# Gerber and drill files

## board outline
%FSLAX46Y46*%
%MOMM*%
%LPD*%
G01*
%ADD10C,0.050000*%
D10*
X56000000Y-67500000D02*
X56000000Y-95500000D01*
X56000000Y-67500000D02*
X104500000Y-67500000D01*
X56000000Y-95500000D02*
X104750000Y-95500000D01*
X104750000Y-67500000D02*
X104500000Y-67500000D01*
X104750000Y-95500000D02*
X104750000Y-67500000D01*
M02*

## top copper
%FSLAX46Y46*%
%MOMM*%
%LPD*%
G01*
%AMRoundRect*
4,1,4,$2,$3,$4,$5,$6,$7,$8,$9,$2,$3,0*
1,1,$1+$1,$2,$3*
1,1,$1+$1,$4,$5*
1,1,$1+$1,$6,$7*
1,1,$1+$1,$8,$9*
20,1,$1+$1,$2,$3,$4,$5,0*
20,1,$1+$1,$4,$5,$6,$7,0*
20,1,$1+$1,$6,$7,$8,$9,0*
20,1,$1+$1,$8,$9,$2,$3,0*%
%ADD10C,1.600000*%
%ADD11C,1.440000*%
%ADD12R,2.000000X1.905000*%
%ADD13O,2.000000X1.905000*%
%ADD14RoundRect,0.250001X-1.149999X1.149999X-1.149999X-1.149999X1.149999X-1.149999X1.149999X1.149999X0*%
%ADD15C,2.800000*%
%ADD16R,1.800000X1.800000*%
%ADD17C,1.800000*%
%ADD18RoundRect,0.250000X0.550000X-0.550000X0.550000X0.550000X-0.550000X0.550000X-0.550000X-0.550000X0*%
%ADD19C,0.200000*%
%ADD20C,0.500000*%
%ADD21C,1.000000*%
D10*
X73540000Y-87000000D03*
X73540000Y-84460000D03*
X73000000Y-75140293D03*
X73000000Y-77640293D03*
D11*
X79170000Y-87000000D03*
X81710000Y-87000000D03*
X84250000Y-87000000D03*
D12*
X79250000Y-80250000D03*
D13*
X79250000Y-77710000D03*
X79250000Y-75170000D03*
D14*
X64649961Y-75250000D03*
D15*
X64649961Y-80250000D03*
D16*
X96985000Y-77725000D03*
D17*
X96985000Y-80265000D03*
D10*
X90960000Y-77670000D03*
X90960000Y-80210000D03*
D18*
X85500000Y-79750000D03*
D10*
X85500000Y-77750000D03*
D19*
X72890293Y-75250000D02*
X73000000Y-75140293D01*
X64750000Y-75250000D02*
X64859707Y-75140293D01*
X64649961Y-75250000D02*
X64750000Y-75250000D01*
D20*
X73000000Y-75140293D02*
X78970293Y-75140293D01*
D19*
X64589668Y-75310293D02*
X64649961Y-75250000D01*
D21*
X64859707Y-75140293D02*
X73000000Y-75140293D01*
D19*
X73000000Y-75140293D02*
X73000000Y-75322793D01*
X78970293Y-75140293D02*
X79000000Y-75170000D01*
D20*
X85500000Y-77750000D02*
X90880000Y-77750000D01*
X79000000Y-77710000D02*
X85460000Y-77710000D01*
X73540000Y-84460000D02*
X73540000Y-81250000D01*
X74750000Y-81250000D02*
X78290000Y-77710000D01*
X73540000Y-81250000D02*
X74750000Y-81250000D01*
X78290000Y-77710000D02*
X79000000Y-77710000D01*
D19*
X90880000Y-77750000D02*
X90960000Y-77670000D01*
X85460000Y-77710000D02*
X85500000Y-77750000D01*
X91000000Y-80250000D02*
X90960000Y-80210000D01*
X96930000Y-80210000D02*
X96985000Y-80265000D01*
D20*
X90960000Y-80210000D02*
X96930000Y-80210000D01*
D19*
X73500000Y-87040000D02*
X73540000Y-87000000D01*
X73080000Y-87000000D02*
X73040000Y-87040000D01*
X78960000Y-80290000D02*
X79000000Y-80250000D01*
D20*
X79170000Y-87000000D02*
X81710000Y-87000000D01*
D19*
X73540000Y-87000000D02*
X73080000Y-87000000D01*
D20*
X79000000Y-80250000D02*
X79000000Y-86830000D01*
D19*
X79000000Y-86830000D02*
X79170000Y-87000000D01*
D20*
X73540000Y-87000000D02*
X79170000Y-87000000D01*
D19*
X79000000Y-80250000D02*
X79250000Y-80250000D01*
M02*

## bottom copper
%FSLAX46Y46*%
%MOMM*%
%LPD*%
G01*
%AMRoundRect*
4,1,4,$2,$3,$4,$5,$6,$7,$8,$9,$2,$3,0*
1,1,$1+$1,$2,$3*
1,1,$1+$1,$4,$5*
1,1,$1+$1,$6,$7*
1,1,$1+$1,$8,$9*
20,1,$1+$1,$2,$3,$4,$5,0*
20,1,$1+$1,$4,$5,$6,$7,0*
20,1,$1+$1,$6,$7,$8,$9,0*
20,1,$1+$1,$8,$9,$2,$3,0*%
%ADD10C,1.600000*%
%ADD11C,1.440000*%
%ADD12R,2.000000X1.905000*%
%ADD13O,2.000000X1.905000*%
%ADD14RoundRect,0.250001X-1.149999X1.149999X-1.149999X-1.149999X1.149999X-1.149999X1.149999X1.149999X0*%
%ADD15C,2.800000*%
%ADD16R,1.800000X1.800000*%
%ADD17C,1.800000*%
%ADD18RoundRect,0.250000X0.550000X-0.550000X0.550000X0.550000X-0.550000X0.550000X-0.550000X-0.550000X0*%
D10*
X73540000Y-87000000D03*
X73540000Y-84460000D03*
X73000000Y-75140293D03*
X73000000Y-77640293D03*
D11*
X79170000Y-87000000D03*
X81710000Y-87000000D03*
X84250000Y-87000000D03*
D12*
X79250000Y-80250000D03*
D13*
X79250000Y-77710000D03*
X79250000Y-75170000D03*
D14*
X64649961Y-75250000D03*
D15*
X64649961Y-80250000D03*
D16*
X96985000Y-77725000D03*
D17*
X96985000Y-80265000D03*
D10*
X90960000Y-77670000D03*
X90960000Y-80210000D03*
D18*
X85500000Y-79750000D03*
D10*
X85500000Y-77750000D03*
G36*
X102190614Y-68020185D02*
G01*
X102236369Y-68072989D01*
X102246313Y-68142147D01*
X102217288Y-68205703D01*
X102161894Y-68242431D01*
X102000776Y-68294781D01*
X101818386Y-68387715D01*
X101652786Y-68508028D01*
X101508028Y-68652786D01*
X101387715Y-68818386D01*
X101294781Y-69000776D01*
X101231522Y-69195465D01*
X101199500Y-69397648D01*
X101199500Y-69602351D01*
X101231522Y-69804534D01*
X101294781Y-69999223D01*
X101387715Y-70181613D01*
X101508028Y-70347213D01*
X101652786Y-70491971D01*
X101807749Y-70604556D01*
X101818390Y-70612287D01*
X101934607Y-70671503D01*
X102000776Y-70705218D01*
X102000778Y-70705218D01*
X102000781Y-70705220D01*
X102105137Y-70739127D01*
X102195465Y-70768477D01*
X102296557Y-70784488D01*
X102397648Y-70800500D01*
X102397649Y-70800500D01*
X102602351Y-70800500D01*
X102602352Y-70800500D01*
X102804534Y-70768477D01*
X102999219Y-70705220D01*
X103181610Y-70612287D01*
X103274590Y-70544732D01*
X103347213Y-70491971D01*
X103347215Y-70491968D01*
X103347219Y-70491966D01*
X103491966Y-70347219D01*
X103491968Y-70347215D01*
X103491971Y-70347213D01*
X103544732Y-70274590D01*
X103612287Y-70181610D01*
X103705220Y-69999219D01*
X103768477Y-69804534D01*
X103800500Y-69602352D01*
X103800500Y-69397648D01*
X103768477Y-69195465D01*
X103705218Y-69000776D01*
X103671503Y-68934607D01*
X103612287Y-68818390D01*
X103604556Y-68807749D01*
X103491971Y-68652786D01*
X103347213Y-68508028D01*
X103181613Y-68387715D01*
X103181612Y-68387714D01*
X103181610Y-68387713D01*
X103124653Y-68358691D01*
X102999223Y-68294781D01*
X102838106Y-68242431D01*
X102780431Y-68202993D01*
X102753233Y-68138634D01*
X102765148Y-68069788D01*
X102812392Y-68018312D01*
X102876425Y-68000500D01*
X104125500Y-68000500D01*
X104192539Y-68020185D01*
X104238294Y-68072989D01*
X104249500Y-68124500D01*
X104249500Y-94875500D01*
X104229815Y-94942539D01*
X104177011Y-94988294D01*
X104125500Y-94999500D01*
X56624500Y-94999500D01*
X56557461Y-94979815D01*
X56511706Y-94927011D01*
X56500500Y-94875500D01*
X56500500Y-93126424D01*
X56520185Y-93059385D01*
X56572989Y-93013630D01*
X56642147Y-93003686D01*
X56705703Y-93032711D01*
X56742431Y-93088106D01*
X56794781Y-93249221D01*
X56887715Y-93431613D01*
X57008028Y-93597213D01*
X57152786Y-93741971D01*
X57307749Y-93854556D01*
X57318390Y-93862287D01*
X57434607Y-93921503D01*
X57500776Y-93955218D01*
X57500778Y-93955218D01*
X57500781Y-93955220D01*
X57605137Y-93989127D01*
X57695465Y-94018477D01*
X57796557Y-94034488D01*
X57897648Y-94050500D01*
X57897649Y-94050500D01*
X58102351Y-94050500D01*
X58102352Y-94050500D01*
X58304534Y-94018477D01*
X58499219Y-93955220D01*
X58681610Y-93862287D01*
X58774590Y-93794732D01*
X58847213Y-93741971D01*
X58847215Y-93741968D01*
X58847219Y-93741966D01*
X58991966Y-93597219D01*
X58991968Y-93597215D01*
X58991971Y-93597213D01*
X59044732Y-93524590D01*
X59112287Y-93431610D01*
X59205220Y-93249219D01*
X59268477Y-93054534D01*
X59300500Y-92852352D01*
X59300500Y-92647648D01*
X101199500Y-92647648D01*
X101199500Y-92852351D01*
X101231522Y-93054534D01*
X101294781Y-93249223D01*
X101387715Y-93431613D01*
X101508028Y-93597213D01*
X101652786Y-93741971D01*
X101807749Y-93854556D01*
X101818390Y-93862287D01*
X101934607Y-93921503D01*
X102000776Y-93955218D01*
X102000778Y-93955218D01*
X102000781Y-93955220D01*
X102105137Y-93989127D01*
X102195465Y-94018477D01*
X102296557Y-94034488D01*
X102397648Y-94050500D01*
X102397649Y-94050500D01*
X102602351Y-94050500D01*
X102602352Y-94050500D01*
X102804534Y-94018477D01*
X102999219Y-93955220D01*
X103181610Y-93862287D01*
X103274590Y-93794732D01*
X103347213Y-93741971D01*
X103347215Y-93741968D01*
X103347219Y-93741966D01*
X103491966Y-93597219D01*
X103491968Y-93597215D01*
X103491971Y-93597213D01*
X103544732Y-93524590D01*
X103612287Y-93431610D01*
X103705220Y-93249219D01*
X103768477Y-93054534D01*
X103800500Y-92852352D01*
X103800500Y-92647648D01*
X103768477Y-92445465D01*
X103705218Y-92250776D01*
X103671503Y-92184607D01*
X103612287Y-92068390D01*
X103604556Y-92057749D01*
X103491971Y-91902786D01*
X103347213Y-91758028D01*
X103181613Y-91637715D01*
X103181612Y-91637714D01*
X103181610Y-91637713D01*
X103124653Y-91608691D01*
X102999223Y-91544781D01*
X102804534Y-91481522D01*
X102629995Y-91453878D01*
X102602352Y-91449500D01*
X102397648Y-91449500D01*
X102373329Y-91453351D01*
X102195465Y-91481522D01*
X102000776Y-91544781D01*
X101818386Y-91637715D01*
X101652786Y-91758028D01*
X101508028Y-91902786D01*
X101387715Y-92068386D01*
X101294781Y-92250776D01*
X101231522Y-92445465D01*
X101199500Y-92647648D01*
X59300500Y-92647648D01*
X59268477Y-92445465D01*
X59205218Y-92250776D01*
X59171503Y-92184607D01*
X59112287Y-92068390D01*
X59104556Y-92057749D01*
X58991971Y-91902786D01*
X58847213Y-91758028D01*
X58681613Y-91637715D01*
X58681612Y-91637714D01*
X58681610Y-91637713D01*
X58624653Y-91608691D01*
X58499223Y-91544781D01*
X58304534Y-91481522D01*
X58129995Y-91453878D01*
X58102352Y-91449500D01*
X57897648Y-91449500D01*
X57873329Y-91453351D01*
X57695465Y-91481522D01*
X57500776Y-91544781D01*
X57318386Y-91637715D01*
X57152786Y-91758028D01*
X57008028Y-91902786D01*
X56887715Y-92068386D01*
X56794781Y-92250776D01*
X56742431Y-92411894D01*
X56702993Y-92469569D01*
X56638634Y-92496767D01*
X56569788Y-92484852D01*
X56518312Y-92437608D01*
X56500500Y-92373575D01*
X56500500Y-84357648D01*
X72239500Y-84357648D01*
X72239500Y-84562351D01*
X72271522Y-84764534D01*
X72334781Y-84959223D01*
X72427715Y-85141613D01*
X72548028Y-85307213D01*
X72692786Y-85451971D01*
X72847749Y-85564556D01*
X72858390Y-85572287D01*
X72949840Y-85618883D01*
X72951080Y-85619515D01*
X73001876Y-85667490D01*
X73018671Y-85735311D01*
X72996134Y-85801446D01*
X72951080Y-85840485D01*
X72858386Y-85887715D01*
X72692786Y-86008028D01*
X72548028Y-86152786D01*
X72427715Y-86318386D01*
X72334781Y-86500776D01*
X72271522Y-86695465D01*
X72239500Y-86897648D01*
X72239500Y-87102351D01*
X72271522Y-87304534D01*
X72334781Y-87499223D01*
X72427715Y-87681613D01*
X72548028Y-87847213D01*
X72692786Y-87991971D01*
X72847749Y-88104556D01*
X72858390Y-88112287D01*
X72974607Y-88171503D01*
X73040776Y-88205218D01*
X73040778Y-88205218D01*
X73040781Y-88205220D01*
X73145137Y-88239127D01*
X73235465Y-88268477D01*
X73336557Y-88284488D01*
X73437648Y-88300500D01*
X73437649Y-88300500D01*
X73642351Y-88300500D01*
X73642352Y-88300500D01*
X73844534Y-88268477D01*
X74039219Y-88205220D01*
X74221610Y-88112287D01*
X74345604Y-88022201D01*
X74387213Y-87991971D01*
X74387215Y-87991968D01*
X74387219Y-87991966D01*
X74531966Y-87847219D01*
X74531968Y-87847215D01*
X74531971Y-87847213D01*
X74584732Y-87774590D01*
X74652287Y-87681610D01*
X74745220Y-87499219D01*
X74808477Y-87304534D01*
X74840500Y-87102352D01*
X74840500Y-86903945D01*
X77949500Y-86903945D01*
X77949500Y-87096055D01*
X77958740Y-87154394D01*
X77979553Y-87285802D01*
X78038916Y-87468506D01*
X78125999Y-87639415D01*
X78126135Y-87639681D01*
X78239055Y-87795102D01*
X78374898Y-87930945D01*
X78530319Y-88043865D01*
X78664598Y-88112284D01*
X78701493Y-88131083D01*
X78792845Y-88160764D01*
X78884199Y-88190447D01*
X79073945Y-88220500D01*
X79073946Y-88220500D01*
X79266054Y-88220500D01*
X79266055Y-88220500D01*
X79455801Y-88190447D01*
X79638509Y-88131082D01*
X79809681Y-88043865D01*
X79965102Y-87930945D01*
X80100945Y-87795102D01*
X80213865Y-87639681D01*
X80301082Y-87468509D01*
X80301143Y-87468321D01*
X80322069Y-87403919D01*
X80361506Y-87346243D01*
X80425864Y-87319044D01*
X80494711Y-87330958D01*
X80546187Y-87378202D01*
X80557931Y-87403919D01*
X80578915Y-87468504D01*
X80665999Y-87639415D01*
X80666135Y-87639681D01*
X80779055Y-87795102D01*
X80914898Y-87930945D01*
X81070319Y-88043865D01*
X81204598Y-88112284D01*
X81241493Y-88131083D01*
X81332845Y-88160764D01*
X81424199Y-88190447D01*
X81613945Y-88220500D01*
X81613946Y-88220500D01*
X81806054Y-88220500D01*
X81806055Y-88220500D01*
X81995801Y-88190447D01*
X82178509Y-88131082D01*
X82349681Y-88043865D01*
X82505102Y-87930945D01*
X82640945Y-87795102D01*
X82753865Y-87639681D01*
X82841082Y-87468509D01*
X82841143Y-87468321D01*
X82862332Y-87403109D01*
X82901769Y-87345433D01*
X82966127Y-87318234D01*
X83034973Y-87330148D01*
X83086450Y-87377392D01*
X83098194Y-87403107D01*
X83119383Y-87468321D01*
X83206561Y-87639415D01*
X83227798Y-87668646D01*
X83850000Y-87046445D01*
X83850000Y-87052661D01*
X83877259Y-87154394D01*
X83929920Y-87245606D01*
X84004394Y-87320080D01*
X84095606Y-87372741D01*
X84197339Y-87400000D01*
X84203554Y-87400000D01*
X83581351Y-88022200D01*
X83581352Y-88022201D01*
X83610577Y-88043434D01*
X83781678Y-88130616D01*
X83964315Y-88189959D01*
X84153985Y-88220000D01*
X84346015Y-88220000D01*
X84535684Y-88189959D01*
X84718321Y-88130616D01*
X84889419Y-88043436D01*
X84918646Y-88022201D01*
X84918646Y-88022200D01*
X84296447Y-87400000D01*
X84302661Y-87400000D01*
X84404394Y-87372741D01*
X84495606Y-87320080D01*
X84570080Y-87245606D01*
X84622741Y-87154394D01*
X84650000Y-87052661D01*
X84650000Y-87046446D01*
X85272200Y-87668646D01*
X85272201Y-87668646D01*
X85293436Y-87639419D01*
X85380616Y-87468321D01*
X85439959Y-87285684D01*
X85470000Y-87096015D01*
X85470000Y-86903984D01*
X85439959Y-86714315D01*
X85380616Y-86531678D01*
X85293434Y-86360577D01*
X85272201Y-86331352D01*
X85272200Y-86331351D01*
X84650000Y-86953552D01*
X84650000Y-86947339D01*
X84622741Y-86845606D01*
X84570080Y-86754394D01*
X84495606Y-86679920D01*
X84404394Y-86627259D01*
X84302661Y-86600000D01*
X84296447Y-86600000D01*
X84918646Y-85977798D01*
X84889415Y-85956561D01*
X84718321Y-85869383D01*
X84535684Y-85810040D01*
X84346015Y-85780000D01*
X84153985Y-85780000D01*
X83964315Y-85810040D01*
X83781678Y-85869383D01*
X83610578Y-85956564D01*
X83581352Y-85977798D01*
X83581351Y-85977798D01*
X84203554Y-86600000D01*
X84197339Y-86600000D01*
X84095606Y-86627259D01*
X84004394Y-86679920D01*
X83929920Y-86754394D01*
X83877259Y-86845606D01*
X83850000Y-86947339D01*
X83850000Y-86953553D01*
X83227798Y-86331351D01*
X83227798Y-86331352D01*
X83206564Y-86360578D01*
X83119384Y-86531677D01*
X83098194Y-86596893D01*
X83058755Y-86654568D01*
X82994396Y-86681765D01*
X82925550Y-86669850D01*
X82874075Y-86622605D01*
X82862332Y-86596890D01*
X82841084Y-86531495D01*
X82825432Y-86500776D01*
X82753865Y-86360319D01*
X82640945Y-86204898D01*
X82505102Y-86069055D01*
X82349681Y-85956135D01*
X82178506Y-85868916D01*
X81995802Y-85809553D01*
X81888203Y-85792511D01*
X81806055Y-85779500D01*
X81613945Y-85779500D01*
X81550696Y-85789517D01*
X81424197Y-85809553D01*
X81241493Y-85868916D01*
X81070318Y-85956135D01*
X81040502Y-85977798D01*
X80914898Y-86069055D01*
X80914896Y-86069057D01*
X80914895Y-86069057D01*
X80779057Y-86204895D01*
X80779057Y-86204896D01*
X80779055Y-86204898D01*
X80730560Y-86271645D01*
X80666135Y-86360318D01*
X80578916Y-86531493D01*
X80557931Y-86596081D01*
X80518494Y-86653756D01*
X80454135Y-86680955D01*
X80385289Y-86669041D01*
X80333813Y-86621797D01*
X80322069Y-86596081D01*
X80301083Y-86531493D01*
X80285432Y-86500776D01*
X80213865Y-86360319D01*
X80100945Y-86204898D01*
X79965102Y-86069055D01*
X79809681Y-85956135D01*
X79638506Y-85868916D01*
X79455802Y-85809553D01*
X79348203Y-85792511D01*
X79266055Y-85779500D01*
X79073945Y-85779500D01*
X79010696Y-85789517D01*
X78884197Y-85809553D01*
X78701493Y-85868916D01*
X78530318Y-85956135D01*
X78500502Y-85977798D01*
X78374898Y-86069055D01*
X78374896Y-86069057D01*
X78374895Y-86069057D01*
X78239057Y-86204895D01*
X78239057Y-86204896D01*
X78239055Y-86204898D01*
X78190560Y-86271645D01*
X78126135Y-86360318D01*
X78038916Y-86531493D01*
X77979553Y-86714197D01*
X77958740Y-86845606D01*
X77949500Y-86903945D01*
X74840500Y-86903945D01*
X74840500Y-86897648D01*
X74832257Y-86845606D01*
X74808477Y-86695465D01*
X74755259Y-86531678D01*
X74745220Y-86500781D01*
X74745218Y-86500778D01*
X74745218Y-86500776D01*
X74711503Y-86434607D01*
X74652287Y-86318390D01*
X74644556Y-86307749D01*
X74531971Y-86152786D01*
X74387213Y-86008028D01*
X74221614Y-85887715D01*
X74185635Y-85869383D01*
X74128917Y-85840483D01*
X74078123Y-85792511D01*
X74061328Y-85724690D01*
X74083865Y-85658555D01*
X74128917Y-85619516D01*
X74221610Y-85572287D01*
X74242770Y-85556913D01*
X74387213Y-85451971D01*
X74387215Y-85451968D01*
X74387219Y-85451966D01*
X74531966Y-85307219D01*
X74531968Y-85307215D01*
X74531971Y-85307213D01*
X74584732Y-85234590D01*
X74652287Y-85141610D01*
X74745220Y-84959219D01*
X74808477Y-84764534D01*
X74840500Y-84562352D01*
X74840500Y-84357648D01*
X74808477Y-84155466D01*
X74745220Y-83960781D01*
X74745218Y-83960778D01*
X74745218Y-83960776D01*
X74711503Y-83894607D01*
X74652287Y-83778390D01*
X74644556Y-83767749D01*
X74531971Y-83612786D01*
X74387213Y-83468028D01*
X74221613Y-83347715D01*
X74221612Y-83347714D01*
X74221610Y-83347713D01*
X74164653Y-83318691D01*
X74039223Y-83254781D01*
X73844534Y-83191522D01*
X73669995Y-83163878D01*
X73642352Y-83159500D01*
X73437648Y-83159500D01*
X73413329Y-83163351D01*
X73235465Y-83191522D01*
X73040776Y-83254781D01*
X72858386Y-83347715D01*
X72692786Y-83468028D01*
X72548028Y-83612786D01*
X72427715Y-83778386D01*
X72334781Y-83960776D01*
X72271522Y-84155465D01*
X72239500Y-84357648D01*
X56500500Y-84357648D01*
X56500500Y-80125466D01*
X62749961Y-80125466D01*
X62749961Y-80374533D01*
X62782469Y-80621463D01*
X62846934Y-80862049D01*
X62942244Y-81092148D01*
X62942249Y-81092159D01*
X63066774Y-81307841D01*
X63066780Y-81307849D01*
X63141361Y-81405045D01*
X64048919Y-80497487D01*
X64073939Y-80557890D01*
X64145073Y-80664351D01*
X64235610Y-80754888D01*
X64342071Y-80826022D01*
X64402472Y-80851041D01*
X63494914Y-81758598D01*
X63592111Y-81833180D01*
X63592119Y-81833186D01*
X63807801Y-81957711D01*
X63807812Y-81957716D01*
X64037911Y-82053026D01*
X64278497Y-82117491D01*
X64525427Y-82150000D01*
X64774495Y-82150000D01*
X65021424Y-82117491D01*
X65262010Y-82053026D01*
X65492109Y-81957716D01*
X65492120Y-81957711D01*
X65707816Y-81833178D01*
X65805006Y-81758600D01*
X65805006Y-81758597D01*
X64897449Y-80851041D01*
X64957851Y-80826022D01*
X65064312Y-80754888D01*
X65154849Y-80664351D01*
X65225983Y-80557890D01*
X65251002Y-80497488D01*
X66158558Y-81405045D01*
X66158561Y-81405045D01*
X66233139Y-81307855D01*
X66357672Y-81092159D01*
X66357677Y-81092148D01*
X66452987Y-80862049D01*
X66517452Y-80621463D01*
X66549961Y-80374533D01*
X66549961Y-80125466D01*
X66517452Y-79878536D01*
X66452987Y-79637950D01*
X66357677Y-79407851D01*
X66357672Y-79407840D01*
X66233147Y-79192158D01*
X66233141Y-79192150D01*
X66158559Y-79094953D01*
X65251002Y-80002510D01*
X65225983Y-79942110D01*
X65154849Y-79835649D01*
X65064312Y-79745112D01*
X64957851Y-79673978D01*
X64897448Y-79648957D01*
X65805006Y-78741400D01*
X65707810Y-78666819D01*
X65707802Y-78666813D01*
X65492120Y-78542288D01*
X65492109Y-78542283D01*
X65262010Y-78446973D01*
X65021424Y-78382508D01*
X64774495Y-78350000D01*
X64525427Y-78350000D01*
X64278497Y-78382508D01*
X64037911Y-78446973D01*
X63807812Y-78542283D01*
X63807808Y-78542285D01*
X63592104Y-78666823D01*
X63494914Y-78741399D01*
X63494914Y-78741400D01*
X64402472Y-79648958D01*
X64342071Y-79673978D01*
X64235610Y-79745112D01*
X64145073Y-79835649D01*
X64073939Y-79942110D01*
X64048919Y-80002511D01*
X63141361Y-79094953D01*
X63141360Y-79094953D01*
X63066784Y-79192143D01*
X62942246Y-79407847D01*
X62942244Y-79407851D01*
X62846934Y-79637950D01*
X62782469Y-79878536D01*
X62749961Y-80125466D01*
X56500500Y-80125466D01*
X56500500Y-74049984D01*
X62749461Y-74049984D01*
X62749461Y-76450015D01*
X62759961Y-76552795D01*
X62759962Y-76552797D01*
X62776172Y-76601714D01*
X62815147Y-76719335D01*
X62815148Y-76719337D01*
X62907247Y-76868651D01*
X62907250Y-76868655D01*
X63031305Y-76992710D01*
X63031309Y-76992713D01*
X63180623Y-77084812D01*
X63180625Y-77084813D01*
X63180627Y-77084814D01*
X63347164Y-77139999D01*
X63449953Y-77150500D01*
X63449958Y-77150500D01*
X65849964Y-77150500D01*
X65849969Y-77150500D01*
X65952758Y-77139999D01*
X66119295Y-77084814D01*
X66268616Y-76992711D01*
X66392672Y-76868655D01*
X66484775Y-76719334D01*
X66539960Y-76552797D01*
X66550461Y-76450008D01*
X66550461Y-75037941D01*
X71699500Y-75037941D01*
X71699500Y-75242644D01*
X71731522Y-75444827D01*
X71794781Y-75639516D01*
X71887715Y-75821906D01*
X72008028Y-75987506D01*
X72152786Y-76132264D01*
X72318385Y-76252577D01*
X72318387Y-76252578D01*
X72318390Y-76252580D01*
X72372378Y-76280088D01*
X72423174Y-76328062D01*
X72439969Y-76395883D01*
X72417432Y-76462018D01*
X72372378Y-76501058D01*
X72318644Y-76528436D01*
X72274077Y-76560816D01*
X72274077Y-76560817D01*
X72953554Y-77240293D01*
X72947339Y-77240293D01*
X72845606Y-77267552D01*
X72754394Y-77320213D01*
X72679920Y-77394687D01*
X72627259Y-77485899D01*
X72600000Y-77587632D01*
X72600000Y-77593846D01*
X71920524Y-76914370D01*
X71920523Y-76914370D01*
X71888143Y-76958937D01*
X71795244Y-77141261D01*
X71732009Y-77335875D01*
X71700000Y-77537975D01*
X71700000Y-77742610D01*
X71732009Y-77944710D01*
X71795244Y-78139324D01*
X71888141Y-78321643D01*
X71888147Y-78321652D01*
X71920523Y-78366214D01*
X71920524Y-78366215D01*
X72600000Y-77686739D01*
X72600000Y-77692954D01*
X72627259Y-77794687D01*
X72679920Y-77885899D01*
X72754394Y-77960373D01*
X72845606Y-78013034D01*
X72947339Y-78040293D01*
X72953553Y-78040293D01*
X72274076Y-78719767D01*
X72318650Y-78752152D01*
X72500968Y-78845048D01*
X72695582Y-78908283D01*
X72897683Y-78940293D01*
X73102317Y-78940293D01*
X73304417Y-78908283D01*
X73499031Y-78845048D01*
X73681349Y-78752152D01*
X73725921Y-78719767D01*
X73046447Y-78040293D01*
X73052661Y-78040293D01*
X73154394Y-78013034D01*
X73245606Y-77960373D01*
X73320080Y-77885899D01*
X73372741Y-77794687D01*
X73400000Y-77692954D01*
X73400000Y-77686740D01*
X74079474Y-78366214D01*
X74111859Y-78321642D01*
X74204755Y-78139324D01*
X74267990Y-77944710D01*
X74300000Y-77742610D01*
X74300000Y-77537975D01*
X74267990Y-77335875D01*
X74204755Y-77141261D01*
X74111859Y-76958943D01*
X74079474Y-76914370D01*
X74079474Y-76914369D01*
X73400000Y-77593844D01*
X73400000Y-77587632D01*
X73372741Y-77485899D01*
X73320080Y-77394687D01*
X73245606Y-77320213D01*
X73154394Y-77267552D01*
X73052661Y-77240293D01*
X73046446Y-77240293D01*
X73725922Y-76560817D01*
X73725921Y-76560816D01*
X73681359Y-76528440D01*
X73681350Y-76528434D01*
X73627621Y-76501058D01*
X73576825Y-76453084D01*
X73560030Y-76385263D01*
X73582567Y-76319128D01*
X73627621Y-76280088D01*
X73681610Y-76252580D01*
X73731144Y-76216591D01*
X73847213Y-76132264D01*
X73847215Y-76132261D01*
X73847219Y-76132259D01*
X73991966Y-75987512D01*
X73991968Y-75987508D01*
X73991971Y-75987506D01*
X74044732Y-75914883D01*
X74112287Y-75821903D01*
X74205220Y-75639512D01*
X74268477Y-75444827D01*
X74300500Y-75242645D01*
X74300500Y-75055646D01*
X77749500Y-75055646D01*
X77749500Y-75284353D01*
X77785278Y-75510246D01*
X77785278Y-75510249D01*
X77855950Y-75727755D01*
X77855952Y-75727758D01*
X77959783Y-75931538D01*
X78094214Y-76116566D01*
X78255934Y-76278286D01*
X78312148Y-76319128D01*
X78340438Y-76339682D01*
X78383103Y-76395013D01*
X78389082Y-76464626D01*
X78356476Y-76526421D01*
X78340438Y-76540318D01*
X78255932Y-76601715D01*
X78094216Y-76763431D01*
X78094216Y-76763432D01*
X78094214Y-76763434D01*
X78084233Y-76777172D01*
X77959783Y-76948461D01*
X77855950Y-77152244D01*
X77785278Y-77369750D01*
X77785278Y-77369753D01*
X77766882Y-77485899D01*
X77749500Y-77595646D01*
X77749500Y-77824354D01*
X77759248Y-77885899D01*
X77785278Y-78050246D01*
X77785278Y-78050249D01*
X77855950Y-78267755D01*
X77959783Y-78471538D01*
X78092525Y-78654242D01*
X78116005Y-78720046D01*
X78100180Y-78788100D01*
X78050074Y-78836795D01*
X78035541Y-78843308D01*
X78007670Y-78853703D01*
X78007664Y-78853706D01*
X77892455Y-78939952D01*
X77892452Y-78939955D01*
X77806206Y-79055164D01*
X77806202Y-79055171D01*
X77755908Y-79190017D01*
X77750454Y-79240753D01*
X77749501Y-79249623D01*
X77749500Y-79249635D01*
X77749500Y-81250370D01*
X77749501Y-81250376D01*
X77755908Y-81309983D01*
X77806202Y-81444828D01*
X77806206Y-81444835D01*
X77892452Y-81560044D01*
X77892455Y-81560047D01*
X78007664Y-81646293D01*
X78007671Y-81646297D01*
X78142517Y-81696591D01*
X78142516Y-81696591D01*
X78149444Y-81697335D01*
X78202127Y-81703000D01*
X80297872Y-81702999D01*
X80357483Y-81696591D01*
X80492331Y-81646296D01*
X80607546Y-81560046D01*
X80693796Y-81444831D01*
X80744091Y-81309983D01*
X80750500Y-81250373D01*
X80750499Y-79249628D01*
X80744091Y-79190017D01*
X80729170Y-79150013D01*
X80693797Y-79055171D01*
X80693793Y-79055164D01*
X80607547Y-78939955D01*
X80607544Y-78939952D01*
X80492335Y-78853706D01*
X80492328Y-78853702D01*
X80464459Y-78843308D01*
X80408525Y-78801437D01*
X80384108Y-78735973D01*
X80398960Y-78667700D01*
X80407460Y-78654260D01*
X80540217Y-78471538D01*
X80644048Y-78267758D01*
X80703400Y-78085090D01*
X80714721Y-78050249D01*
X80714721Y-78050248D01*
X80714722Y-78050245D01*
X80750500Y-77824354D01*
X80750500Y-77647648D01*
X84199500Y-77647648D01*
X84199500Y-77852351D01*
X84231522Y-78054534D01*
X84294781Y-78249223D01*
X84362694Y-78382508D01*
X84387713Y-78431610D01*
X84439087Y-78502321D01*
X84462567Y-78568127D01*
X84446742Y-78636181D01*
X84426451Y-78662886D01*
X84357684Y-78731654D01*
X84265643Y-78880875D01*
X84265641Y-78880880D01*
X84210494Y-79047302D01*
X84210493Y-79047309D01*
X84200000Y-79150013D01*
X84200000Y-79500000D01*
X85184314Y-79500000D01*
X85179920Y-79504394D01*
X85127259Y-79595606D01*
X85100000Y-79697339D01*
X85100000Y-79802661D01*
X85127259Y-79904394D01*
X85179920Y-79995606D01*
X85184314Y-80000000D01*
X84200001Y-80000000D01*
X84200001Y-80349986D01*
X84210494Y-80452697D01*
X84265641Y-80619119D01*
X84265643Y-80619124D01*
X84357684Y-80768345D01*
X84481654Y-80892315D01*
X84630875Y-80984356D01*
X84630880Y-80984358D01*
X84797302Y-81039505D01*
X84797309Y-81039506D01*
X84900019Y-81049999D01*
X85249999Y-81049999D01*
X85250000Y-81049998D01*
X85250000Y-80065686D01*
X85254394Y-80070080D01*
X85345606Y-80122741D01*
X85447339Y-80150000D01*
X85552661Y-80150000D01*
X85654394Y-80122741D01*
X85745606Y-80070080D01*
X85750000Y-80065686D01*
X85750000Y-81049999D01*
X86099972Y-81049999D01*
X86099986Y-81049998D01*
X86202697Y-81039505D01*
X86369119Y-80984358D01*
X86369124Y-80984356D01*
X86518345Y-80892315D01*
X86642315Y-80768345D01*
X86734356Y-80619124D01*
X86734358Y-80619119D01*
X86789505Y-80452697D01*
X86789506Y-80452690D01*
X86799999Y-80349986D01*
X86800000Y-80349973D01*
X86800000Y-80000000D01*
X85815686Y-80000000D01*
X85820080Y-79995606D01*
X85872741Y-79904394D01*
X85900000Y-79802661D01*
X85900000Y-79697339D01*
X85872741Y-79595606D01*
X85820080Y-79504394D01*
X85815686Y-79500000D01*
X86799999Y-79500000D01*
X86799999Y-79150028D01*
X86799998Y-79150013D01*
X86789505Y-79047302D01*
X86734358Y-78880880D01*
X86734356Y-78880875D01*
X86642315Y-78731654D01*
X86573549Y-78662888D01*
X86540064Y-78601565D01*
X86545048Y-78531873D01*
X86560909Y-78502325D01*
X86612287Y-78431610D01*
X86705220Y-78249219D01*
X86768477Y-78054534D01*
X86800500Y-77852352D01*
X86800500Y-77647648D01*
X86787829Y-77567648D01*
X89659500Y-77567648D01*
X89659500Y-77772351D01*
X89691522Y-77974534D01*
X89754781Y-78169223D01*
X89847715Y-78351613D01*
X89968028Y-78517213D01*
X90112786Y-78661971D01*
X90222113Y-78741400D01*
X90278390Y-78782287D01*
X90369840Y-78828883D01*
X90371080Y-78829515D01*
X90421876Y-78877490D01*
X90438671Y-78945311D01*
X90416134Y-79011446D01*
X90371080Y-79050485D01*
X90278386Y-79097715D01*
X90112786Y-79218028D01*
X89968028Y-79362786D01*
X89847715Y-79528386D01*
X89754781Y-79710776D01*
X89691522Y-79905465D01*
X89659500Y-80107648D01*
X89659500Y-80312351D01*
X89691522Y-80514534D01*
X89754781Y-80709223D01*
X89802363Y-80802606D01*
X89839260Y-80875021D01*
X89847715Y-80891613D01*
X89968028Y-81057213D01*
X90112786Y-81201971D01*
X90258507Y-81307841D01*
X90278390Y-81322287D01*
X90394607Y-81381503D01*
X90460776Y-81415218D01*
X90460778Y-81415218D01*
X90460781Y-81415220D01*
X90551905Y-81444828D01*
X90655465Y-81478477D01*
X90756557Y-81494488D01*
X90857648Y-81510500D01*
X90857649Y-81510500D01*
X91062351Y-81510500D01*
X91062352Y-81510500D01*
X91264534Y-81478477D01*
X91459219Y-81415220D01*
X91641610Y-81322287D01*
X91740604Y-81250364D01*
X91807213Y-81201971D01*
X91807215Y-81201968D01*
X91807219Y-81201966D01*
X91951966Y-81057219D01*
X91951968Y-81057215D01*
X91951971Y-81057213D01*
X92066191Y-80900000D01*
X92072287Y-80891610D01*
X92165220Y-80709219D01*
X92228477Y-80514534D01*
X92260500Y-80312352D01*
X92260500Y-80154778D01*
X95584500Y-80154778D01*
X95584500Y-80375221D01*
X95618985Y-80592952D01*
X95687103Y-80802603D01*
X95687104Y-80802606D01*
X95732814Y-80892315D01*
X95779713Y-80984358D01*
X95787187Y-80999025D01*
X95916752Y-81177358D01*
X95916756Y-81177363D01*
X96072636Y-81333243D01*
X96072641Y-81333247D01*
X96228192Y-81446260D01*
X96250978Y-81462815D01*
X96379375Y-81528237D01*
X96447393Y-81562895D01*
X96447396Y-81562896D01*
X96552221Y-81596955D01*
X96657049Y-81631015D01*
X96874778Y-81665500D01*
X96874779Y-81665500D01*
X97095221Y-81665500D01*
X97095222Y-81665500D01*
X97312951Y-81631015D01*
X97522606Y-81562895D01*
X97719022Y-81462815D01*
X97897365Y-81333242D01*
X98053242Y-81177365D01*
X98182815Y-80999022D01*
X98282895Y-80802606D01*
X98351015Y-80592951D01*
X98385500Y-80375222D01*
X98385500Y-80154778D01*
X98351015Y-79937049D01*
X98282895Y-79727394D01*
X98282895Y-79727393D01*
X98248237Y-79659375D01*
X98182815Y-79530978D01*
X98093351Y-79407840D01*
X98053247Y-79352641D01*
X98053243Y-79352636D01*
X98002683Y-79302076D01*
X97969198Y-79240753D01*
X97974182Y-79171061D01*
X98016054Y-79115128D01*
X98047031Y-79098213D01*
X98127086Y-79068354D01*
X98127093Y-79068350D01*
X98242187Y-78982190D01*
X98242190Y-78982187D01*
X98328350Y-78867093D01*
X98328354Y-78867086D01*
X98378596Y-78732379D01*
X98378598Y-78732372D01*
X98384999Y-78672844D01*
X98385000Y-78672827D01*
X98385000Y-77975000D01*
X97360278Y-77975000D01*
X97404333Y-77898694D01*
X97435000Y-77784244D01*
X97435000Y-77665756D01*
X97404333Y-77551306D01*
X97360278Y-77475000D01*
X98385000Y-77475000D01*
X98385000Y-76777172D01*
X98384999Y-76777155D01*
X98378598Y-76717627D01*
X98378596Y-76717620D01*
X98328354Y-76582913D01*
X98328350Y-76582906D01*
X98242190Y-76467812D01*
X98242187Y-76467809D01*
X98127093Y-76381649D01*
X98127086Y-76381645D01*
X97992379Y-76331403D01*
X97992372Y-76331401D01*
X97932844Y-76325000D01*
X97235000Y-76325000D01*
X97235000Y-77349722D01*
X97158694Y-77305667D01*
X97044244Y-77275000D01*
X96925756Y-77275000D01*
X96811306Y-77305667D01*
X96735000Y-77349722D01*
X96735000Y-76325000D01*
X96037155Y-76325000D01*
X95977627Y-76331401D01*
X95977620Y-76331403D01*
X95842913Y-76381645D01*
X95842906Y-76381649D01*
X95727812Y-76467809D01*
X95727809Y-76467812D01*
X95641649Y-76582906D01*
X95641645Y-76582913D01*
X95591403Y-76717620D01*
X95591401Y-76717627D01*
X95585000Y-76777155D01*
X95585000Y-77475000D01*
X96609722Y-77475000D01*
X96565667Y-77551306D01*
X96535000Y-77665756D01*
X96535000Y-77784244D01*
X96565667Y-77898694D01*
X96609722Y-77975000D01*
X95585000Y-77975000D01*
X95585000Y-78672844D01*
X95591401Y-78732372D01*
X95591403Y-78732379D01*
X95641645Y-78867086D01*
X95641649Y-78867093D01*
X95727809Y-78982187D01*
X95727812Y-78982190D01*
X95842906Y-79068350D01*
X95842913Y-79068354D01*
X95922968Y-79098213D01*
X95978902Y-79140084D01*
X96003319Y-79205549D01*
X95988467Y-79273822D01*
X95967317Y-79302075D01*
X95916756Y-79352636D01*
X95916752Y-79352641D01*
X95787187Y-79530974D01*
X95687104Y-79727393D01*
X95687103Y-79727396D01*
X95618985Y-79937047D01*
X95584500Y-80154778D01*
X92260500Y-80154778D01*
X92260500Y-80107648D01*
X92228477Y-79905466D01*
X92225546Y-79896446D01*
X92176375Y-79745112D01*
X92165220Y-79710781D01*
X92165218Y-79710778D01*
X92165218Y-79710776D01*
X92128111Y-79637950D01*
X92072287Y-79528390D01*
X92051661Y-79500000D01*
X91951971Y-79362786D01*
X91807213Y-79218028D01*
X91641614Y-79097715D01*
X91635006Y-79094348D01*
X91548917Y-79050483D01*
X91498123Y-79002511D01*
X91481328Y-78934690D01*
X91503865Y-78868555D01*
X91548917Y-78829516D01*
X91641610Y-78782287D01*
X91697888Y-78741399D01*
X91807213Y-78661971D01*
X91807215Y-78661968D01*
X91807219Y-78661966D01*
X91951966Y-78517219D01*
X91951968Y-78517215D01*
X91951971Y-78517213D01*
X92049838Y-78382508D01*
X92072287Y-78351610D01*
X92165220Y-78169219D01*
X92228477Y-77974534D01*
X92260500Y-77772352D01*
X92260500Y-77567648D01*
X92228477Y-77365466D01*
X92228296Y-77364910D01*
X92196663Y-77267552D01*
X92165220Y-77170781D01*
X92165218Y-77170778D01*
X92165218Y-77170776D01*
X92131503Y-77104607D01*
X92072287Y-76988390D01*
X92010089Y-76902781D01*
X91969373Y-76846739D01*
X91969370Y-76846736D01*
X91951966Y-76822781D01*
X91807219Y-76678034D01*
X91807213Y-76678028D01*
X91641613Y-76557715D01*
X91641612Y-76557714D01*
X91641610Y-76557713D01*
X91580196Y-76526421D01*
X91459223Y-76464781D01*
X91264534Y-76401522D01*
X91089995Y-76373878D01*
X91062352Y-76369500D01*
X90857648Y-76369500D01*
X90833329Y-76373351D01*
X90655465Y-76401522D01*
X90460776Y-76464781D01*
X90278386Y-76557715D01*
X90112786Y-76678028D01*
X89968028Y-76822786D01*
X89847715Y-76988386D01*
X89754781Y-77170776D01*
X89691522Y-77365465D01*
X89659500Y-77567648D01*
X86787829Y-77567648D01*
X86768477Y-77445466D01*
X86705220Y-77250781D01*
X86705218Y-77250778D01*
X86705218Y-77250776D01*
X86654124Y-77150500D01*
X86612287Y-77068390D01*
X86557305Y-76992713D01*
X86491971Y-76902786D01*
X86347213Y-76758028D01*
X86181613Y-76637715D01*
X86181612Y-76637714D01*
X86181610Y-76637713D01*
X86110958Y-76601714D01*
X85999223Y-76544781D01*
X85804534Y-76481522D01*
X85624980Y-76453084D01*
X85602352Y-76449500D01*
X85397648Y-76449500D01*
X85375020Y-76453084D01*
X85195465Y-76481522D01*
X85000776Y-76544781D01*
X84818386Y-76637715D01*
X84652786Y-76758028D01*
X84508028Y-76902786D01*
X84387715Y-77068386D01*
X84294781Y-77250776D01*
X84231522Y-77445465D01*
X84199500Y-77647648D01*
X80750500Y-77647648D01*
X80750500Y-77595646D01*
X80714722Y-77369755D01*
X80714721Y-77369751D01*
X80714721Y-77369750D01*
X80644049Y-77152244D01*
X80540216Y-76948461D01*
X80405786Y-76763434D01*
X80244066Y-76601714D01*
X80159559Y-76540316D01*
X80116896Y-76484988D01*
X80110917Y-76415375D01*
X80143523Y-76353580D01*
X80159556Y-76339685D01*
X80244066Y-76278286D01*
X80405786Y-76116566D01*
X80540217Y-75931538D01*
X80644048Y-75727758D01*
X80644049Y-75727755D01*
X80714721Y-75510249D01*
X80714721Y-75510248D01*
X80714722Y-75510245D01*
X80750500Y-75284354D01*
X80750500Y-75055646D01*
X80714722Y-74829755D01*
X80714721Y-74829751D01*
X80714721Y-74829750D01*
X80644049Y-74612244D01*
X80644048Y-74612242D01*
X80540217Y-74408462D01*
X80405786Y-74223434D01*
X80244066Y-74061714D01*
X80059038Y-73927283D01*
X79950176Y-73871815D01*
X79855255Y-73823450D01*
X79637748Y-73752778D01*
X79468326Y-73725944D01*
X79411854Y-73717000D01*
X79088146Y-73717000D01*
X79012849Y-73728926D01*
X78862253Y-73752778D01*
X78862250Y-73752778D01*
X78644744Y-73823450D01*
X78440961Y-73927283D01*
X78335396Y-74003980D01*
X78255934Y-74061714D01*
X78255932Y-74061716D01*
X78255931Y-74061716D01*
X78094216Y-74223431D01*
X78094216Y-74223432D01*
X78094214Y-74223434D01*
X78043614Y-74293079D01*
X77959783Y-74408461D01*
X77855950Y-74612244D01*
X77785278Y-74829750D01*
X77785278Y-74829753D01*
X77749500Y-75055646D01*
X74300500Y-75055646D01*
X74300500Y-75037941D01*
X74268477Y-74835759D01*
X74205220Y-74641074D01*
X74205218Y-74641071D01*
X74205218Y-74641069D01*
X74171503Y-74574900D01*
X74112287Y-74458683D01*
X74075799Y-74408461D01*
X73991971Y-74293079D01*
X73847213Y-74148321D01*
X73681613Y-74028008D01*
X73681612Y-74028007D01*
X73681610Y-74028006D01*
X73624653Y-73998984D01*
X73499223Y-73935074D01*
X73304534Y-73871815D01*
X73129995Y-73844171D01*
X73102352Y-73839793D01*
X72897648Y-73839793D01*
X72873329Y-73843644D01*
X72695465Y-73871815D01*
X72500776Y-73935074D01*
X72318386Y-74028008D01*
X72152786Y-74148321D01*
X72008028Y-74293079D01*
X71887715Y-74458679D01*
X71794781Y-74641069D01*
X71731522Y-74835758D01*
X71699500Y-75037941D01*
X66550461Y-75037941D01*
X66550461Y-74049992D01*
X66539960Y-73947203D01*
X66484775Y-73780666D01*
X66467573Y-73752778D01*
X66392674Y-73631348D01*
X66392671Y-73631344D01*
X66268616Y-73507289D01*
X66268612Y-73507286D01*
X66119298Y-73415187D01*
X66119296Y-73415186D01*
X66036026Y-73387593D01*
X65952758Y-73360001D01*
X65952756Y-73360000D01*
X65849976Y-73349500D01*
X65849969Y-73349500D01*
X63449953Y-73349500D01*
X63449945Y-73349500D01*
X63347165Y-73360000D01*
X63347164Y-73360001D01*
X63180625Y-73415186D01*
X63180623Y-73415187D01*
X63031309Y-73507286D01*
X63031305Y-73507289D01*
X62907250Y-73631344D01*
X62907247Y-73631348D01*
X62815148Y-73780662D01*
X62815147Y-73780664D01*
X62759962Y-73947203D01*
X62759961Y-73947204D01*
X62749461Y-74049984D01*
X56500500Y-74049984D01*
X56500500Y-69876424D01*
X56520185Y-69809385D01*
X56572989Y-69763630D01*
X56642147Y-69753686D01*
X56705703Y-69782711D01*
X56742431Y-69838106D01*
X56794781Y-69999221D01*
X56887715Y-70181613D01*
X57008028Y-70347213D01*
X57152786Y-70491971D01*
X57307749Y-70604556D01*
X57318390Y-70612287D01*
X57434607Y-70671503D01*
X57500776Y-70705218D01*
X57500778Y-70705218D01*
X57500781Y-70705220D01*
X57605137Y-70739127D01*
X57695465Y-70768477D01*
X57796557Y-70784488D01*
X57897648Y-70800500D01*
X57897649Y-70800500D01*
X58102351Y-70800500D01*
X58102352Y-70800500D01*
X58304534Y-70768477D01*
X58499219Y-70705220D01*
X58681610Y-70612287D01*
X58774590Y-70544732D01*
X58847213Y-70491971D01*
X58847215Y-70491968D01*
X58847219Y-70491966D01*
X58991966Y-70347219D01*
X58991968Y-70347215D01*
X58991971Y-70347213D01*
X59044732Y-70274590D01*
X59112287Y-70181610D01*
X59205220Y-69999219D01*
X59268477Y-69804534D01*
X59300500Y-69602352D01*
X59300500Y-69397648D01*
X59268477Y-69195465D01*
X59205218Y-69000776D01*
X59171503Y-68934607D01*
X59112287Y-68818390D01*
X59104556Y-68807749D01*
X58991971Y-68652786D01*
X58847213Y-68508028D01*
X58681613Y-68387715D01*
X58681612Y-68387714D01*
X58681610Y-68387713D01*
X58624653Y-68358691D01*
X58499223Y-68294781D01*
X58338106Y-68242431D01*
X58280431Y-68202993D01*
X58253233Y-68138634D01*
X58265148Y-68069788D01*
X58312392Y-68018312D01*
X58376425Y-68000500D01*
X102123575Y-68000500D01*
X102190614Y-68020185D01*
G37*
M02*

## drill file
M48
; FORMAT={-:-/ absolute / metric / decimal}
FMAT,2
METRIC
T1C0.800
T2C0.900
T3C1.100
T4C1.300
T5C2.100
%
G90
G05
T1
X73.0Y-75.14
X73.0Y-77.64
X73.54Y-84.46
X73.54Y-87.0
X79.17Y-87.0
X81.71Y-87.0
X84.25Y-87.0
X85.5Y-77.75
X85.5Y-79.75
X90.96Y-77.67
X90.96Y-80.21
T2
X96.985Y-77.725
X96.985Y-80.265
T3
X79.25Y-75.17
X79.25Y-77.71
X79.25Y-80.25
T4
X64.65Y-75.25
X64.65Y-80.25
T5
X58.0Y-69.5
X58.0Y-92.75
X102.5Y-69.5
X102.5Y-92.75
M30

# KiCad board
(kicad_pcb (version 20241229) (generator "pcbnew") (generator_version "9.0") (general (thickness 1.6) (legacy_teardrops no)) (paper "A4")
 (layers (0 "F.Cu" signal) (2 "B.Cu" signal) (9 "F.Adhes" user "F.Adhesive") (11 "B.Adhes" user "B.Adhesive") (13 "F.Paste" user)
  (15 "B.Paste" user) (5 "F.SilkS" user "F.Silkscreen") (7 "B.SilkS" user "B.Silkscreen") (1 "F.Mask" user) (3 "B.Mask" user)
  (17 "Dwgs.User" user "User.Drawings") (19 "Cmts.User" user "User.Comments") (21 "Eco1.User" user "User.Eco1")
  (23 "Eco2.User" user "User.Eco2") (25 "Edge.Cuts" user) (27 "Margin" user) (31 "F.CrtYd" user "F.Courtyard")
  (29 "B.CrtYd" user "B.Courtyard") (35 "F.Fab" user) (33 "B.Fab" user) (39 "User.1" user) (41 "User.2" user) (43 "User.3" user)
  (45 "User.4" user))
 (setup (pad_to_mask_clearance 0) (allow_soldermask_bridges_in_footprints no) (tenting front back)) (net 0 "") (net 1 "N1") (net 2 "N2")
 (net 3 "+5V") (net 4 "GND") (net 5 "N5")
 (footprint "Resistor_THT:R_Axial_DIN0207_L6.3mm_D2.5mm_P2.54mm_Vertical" (layer "F.Cu") (at 73.54 87 90)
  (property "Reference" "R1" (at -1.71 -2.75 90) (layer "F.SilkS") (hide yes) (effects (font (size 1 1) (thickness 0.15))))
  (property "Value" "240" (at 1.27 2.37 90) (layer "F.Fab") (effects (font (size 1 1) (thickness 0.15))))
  (pad "1" thru_hole circle (at 0 0 90) (size 1.6 1.6) (drill 0.8) (layers "*.Cu" "*.Mask") (remove_unused_layers no) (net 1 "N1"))
  (pad "2" thru_hole circle (at 2.54 0 90) (size 1.6 1.6) (drill 0.8) (layers "*.Cu" "*.Mask") (remove_unused_layers no) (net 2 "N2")))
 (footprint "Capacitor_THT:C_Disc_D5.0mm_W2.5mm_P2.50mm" (layer "F.Cu") (at 73 75.140293 -90)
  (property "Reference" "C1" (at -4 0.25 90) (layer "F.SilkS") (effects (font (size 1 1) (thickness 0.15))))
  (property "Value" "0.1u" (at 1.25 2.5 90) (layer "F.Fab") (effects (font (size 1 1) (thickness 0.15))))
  (pad "1" thru_hole circle (at 0 0 270) (size 1.6 1.6) (drill 0.8) (layers "*.Cu" "*.Mask") (remove_unused_layers no) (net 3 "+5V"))
  (pad "2" thru_hole circle (at 2.5 0 270) (size 1.6 1.6) (drill 0.8) (layers "*.Cu" "*.Mask") (remove_unused_layers no) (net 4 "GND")))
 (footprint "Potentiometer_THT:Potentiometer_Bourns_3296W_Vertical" (layer "F.Cu") (at 79.17 87 180)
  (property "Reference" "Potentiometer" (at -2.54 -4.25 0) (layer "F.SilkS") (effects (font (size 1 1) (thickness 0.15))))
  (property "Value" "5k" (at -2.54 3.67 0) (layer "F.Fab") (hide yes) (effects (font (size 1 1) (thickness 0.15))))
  (pad "1" thru_hole circle (at 0 0 180) (size 1.44 1.44) (drill 0.8) (layers "*.Cu" "*.Mask") (remove_unused_layers no) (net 1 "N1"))
  (pad "2" thru_hole circle (at -2.54 0 180) (size 1.44 1.44) (drill 0.8) (layers "*.Cu" "*.Mask") (remove_unused_layers no) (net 1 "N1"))
  (pad "3" thru_hole circle (at -5.08 0 180) (size 1.44 1.44) (drill 0.8) (layers "*.Cu" "*.Mask") (remove_unused_layers no) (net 4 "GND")))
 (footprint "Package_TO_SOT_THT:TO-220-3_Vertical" (layer "F.Cu") (at 79.25 80.25 90)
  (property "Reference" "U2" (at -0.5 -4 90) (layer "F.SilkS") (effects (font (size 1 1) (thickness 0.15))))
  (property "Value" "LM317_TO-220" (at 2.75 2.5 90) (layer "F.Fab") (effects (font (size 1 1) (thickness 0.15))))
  (pad "1" thru_hole rect (at 0 0 90) (size 1.905 2) (drill 1.1) (layers "*.Cu" "*.Mask") (remove_unused_layers no) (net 1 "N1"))
  (pad "2" thru_hole oval (at 2.54 0 90) (size 1.905 2) (drill 1.1) (layers "*.Cu" "*.Mask") (remove_unused_layers no) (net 2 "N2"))
  (pad "3" thru_hole oval (at 5.08 0 90) (size 1.905 2) (drill 1.1) (layers "*.Cu" "*.Mask") (remove_unused_layers no) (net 3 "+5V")))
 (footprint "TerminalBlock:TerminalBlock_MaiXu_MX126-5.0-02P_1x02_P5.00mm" (layer "F.Cu") (at 64.649961 75.25 -90)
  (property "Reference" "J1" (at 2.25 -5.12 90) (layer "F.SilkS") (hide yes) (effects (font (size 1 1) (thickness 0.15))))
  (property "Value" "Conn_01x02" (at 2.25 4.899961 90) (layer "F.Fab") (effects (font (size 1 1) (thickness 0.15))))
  (pad "1" thru_hole roundrect (at 0 0 270) (size 2.8 2.8) (drill 1.3) (layers "*.Cu" "*.Mask") (remove_unused_layers no)
   (roundrect_rratio 0.089286) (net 3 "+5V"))
  (pad "2" thru_hole circle (at 5 0 270) (size 2.8 2.8) (drill 1.3) (layers "*.Cu" "*.Mask") (remove_unused_layers no) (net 4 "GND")))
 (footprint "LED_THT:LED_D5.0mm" (layer "F.Cu") (at 96.985 77.725 -90)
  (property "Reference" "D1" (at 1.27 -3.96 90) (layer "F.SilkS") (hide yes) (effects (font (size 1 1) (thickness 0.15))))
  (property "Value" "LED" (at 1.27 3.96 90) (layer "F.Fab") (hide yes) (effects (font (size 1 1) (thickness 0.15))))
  (pad "1" thru_hole rect (at 0 0 270) (size 1.8 1.8) (drill 0.9) (layers "*.Cu" "*.Mask") (remove_unused_layers no) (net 4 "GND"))
  (pad "2" thru_hole circle (at 2.54 0 270) (size 1.8 1.8) (drill 0.9) (layers "*.Cu" "*.Mask") (remove_unused_layers no) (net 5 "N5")))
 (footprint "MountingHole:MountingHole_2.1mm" (layer "F.Cu") (at 58 92.75)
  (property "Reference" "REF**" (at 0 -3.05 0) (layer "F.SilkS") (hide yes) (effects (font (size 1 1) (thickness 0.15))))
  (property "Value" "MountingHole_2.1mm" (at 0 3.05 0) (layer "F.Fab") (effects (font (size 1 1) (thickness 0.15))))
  (pad "" np_thru_hole circle (at 0 0) (size 2.1 2.1) (drill 2.1) (layers "*.Cu" "*.Mask")))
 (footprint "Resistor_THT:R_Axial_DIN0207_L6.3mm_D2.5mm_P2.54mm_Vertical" (layer "F.Cu") (at 90.96 77.67 -90)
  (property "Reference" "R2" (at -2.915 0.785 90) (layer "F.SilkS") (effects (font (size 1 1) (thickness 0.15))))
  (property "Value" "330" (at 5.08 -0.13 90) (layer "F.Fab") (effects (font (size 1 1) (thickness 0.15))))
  (pad "1" thru_hole circle (at 0 0 270) (size 1.6 1.6) (drill 0.8) (layers "*.Cu" "*.Mask") (remove_unused_layers no) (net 2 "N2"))
  (pad "2" thru_hole circle (at 2.54 0 270) (size 1.6 1.6) (drill 0.8) (layers "*.Cu" "*.Mask") (remove_unused_layers no) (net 5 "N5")))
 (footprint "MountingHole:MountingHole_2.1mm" (layer "F.Cu") (at 102.5 92.75)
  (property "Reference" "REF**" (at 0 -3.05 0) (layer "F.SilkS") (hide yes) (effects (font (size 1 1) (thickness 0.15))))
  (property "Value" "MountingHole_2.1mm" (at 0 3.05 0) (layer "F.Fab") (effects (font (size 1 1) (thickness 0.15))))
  (pad "" np_thru_hole circle (at 0 0) (size 2.1 2.1) (drill 2.1) (layers "*.Cu" "*.Mask")))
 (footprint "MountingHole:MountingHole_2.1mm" (layer "F.Cu") (at 102.5 69.5)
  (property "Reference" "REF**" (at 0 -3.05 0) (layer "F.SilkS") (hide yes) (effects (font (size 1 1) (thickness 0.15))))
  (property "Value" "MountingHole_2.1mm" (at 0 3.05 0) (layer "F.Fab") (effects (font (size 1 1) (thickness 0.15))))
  (pad "" np_thru_hole circle (at 0 0) (size 2.1 2.1) (drill 2.1) (layers "*.Cu" "*.Mask")))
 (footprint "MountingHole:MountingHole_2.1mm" (layer "F.Cu") (at 58 69.5)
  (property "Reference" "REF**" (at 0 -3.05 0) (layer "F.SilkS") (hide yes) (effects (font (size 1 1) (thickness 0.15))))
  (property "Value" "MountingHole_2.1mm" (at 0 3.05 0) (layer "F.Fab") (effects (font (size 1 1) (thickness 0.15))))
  (pad "" np_thru_hole circle (at 0 0) (size 2.1 2.1) (drill 2.1) (layers "*.Cu" "*.Mask")))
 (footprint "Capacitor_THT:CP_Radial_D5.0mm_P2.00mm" (layer "F.Cu") (at 85.5 79.75 90)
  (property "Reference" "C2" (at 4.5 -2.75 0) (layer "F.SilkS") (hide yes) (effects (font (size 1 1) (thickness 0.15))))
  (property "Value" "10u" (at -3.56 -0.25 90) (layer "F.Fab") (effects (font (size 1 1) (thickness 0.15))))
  (pad "1" thru_hole roundrect (at 0 0 90) (size 1.6 1.6) (drill 0.8) (layers "*.Cu" "*.Mask") (remove_unused_layers no)
   (roundrect_rratio 0.15625) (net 4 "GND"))
  (pad "2" thru_hole circle (at 2 0 90) (size 1.6 1.6) (drill 0.8) (layers "*.Cu" "*.Mask") (remove_unused_layers no) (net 2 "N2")))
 (gr_line (start 56 67.5) (end 56 95.5) (stroke (width 0.05) (type default)) (layer "Edge.Cuts"))
 (gr_line (start 56 67.5) (end 104.5 67.5) (stroke (width 0.05) (type default)) (layer "Edge.Cuts"))
 (gr_line (start 56 95.5) (end 104.75 95.5) (stroke (width 0.05) (type default)) (layer "Edge.Cuts"))
 (gr_line (start 104.75 67.5) (end 104.5 67.5) (stroke (width 0.05) (type default)) (layer "Edge.Cuts"))
 (gr_line (start 104.75 95.5) (end 104.75 67.5) (stroke (width 0.05) (type default)) (layer "Edge.Cuts"))
 (segment (start 72.890293 75.25) (end 73 75.140293) (width 0.2) (layer "F.Cu") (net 3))
 (segment (start 64.75 75.25) (end 64.859707 75.140293) (width 0.2) (layer "F.Cu") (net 3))
 (segment (start 64.649961 75.25) (end 64.75 75.25) (width 0.2) (layer "F.Cu") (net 3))
 (segment (start 73 75.140293) (end 78.970293 75.140293) (width 0.5) (layer "F.Cu") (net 3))
 (segment (start 64.589668 75.310293) (end 64.649961 75.25) (width 0.2) (layer "F.Cu") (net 3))
 (segment (start 64.859707 75.140293) (end 73 75.140293) (width 1) (layer "F.Cu") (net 3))
 (segment (start 73 75.140293) (end 73 75.322793) (width 0.2) (layer "F.Cu") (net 3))
 (segment (start 78.970293 75.140293) (end 79 75.17) (width 0.2) (layer "F.Cu") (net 3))
 (segment (start 85.5 77.75) (end 90.88 77.75) (width 0.5) (layer "F.Cu") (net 2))
 (segment (start 79 77.71) (end 85.46 77.71) (width 0.5) (layer "F.Cu") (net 2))
 (segment (start 73.54 84.46) (end 73.54 81.25) (width 0.5) (layer "F.Cu") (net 2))
 (segment (start 74.75 81.25) (end 78.29 77.71) (width 0.5) (layer "F.Cu") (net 2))
 (segment (start 73.54 81.25) (end 74.75 81.25) (width 0.5) (layer "F.Cu") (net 2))
 (segment (start 78.29 77.71) (end 79 77.71) (width 0.5) (layer "F.Cu") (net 2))
 (segment (start 90.88 77.75) (end 90.96 77.67) (width 0.2) (layer "F.Cu") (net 2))
 (segment (start 85.46 77.71) (end 85.5 77.75) (width 0.2) (layer "F.Cu") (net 2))
 (segment (start 91 80.25) (end 90.96 80.21) (width 0.2) (layer "F.Cu") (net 5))
 (segment (start 96.93 80.21) (end 96.985 80.265) (width 0.2) (layer "F.Cu") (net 5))
 (segment (start 90.96 80.21) (end 96.93 80.21) (width 0.5) (layer "F.Cu") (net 5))
 (segment (start 73.5 87.04) (end 73.54 87) (width 0.2) (layer "F.Cu") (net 1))
 (segment (start 73.08 87) (end 73.04 87.04) (width 0.2) (layer "F.Cu") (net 1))
 (segment (start 78.96 80.29) (end 79 80.25) (width 0.2) (layer "F.Cu") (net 1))
 (segment (start 79.17 87) (end 81.71 87) (width 0.5) (layer "F.Cu") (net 1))
 (segment (start 73.54 87) (end 73.08 87) (width 0.2) (layer "F.Cu") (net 1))
 (segment (start 79 80.25) (end 79 86.83) (width 0.5) (layer "F.Cu") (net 1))
 (segment (start 79 86.83) (end 79.17 87) (width 0.2) (layer "F.Cu") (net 1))
 (segment (start 73.54 87) (end 79.17 87) (width 0.5) (layer "F.Cu") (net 1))
 (segment (start 79 80.25) (end 79.25 80.25) (width 0.2) (layer "F.Cu") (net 1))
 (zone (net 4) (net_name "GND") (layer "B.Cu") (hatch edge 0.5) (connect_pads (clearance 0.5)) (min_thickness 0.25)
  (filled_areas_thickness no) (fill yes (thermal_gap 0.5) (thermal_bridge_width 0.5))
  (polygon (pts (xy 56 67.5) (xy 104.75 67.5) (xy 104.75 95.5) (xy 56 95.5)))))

